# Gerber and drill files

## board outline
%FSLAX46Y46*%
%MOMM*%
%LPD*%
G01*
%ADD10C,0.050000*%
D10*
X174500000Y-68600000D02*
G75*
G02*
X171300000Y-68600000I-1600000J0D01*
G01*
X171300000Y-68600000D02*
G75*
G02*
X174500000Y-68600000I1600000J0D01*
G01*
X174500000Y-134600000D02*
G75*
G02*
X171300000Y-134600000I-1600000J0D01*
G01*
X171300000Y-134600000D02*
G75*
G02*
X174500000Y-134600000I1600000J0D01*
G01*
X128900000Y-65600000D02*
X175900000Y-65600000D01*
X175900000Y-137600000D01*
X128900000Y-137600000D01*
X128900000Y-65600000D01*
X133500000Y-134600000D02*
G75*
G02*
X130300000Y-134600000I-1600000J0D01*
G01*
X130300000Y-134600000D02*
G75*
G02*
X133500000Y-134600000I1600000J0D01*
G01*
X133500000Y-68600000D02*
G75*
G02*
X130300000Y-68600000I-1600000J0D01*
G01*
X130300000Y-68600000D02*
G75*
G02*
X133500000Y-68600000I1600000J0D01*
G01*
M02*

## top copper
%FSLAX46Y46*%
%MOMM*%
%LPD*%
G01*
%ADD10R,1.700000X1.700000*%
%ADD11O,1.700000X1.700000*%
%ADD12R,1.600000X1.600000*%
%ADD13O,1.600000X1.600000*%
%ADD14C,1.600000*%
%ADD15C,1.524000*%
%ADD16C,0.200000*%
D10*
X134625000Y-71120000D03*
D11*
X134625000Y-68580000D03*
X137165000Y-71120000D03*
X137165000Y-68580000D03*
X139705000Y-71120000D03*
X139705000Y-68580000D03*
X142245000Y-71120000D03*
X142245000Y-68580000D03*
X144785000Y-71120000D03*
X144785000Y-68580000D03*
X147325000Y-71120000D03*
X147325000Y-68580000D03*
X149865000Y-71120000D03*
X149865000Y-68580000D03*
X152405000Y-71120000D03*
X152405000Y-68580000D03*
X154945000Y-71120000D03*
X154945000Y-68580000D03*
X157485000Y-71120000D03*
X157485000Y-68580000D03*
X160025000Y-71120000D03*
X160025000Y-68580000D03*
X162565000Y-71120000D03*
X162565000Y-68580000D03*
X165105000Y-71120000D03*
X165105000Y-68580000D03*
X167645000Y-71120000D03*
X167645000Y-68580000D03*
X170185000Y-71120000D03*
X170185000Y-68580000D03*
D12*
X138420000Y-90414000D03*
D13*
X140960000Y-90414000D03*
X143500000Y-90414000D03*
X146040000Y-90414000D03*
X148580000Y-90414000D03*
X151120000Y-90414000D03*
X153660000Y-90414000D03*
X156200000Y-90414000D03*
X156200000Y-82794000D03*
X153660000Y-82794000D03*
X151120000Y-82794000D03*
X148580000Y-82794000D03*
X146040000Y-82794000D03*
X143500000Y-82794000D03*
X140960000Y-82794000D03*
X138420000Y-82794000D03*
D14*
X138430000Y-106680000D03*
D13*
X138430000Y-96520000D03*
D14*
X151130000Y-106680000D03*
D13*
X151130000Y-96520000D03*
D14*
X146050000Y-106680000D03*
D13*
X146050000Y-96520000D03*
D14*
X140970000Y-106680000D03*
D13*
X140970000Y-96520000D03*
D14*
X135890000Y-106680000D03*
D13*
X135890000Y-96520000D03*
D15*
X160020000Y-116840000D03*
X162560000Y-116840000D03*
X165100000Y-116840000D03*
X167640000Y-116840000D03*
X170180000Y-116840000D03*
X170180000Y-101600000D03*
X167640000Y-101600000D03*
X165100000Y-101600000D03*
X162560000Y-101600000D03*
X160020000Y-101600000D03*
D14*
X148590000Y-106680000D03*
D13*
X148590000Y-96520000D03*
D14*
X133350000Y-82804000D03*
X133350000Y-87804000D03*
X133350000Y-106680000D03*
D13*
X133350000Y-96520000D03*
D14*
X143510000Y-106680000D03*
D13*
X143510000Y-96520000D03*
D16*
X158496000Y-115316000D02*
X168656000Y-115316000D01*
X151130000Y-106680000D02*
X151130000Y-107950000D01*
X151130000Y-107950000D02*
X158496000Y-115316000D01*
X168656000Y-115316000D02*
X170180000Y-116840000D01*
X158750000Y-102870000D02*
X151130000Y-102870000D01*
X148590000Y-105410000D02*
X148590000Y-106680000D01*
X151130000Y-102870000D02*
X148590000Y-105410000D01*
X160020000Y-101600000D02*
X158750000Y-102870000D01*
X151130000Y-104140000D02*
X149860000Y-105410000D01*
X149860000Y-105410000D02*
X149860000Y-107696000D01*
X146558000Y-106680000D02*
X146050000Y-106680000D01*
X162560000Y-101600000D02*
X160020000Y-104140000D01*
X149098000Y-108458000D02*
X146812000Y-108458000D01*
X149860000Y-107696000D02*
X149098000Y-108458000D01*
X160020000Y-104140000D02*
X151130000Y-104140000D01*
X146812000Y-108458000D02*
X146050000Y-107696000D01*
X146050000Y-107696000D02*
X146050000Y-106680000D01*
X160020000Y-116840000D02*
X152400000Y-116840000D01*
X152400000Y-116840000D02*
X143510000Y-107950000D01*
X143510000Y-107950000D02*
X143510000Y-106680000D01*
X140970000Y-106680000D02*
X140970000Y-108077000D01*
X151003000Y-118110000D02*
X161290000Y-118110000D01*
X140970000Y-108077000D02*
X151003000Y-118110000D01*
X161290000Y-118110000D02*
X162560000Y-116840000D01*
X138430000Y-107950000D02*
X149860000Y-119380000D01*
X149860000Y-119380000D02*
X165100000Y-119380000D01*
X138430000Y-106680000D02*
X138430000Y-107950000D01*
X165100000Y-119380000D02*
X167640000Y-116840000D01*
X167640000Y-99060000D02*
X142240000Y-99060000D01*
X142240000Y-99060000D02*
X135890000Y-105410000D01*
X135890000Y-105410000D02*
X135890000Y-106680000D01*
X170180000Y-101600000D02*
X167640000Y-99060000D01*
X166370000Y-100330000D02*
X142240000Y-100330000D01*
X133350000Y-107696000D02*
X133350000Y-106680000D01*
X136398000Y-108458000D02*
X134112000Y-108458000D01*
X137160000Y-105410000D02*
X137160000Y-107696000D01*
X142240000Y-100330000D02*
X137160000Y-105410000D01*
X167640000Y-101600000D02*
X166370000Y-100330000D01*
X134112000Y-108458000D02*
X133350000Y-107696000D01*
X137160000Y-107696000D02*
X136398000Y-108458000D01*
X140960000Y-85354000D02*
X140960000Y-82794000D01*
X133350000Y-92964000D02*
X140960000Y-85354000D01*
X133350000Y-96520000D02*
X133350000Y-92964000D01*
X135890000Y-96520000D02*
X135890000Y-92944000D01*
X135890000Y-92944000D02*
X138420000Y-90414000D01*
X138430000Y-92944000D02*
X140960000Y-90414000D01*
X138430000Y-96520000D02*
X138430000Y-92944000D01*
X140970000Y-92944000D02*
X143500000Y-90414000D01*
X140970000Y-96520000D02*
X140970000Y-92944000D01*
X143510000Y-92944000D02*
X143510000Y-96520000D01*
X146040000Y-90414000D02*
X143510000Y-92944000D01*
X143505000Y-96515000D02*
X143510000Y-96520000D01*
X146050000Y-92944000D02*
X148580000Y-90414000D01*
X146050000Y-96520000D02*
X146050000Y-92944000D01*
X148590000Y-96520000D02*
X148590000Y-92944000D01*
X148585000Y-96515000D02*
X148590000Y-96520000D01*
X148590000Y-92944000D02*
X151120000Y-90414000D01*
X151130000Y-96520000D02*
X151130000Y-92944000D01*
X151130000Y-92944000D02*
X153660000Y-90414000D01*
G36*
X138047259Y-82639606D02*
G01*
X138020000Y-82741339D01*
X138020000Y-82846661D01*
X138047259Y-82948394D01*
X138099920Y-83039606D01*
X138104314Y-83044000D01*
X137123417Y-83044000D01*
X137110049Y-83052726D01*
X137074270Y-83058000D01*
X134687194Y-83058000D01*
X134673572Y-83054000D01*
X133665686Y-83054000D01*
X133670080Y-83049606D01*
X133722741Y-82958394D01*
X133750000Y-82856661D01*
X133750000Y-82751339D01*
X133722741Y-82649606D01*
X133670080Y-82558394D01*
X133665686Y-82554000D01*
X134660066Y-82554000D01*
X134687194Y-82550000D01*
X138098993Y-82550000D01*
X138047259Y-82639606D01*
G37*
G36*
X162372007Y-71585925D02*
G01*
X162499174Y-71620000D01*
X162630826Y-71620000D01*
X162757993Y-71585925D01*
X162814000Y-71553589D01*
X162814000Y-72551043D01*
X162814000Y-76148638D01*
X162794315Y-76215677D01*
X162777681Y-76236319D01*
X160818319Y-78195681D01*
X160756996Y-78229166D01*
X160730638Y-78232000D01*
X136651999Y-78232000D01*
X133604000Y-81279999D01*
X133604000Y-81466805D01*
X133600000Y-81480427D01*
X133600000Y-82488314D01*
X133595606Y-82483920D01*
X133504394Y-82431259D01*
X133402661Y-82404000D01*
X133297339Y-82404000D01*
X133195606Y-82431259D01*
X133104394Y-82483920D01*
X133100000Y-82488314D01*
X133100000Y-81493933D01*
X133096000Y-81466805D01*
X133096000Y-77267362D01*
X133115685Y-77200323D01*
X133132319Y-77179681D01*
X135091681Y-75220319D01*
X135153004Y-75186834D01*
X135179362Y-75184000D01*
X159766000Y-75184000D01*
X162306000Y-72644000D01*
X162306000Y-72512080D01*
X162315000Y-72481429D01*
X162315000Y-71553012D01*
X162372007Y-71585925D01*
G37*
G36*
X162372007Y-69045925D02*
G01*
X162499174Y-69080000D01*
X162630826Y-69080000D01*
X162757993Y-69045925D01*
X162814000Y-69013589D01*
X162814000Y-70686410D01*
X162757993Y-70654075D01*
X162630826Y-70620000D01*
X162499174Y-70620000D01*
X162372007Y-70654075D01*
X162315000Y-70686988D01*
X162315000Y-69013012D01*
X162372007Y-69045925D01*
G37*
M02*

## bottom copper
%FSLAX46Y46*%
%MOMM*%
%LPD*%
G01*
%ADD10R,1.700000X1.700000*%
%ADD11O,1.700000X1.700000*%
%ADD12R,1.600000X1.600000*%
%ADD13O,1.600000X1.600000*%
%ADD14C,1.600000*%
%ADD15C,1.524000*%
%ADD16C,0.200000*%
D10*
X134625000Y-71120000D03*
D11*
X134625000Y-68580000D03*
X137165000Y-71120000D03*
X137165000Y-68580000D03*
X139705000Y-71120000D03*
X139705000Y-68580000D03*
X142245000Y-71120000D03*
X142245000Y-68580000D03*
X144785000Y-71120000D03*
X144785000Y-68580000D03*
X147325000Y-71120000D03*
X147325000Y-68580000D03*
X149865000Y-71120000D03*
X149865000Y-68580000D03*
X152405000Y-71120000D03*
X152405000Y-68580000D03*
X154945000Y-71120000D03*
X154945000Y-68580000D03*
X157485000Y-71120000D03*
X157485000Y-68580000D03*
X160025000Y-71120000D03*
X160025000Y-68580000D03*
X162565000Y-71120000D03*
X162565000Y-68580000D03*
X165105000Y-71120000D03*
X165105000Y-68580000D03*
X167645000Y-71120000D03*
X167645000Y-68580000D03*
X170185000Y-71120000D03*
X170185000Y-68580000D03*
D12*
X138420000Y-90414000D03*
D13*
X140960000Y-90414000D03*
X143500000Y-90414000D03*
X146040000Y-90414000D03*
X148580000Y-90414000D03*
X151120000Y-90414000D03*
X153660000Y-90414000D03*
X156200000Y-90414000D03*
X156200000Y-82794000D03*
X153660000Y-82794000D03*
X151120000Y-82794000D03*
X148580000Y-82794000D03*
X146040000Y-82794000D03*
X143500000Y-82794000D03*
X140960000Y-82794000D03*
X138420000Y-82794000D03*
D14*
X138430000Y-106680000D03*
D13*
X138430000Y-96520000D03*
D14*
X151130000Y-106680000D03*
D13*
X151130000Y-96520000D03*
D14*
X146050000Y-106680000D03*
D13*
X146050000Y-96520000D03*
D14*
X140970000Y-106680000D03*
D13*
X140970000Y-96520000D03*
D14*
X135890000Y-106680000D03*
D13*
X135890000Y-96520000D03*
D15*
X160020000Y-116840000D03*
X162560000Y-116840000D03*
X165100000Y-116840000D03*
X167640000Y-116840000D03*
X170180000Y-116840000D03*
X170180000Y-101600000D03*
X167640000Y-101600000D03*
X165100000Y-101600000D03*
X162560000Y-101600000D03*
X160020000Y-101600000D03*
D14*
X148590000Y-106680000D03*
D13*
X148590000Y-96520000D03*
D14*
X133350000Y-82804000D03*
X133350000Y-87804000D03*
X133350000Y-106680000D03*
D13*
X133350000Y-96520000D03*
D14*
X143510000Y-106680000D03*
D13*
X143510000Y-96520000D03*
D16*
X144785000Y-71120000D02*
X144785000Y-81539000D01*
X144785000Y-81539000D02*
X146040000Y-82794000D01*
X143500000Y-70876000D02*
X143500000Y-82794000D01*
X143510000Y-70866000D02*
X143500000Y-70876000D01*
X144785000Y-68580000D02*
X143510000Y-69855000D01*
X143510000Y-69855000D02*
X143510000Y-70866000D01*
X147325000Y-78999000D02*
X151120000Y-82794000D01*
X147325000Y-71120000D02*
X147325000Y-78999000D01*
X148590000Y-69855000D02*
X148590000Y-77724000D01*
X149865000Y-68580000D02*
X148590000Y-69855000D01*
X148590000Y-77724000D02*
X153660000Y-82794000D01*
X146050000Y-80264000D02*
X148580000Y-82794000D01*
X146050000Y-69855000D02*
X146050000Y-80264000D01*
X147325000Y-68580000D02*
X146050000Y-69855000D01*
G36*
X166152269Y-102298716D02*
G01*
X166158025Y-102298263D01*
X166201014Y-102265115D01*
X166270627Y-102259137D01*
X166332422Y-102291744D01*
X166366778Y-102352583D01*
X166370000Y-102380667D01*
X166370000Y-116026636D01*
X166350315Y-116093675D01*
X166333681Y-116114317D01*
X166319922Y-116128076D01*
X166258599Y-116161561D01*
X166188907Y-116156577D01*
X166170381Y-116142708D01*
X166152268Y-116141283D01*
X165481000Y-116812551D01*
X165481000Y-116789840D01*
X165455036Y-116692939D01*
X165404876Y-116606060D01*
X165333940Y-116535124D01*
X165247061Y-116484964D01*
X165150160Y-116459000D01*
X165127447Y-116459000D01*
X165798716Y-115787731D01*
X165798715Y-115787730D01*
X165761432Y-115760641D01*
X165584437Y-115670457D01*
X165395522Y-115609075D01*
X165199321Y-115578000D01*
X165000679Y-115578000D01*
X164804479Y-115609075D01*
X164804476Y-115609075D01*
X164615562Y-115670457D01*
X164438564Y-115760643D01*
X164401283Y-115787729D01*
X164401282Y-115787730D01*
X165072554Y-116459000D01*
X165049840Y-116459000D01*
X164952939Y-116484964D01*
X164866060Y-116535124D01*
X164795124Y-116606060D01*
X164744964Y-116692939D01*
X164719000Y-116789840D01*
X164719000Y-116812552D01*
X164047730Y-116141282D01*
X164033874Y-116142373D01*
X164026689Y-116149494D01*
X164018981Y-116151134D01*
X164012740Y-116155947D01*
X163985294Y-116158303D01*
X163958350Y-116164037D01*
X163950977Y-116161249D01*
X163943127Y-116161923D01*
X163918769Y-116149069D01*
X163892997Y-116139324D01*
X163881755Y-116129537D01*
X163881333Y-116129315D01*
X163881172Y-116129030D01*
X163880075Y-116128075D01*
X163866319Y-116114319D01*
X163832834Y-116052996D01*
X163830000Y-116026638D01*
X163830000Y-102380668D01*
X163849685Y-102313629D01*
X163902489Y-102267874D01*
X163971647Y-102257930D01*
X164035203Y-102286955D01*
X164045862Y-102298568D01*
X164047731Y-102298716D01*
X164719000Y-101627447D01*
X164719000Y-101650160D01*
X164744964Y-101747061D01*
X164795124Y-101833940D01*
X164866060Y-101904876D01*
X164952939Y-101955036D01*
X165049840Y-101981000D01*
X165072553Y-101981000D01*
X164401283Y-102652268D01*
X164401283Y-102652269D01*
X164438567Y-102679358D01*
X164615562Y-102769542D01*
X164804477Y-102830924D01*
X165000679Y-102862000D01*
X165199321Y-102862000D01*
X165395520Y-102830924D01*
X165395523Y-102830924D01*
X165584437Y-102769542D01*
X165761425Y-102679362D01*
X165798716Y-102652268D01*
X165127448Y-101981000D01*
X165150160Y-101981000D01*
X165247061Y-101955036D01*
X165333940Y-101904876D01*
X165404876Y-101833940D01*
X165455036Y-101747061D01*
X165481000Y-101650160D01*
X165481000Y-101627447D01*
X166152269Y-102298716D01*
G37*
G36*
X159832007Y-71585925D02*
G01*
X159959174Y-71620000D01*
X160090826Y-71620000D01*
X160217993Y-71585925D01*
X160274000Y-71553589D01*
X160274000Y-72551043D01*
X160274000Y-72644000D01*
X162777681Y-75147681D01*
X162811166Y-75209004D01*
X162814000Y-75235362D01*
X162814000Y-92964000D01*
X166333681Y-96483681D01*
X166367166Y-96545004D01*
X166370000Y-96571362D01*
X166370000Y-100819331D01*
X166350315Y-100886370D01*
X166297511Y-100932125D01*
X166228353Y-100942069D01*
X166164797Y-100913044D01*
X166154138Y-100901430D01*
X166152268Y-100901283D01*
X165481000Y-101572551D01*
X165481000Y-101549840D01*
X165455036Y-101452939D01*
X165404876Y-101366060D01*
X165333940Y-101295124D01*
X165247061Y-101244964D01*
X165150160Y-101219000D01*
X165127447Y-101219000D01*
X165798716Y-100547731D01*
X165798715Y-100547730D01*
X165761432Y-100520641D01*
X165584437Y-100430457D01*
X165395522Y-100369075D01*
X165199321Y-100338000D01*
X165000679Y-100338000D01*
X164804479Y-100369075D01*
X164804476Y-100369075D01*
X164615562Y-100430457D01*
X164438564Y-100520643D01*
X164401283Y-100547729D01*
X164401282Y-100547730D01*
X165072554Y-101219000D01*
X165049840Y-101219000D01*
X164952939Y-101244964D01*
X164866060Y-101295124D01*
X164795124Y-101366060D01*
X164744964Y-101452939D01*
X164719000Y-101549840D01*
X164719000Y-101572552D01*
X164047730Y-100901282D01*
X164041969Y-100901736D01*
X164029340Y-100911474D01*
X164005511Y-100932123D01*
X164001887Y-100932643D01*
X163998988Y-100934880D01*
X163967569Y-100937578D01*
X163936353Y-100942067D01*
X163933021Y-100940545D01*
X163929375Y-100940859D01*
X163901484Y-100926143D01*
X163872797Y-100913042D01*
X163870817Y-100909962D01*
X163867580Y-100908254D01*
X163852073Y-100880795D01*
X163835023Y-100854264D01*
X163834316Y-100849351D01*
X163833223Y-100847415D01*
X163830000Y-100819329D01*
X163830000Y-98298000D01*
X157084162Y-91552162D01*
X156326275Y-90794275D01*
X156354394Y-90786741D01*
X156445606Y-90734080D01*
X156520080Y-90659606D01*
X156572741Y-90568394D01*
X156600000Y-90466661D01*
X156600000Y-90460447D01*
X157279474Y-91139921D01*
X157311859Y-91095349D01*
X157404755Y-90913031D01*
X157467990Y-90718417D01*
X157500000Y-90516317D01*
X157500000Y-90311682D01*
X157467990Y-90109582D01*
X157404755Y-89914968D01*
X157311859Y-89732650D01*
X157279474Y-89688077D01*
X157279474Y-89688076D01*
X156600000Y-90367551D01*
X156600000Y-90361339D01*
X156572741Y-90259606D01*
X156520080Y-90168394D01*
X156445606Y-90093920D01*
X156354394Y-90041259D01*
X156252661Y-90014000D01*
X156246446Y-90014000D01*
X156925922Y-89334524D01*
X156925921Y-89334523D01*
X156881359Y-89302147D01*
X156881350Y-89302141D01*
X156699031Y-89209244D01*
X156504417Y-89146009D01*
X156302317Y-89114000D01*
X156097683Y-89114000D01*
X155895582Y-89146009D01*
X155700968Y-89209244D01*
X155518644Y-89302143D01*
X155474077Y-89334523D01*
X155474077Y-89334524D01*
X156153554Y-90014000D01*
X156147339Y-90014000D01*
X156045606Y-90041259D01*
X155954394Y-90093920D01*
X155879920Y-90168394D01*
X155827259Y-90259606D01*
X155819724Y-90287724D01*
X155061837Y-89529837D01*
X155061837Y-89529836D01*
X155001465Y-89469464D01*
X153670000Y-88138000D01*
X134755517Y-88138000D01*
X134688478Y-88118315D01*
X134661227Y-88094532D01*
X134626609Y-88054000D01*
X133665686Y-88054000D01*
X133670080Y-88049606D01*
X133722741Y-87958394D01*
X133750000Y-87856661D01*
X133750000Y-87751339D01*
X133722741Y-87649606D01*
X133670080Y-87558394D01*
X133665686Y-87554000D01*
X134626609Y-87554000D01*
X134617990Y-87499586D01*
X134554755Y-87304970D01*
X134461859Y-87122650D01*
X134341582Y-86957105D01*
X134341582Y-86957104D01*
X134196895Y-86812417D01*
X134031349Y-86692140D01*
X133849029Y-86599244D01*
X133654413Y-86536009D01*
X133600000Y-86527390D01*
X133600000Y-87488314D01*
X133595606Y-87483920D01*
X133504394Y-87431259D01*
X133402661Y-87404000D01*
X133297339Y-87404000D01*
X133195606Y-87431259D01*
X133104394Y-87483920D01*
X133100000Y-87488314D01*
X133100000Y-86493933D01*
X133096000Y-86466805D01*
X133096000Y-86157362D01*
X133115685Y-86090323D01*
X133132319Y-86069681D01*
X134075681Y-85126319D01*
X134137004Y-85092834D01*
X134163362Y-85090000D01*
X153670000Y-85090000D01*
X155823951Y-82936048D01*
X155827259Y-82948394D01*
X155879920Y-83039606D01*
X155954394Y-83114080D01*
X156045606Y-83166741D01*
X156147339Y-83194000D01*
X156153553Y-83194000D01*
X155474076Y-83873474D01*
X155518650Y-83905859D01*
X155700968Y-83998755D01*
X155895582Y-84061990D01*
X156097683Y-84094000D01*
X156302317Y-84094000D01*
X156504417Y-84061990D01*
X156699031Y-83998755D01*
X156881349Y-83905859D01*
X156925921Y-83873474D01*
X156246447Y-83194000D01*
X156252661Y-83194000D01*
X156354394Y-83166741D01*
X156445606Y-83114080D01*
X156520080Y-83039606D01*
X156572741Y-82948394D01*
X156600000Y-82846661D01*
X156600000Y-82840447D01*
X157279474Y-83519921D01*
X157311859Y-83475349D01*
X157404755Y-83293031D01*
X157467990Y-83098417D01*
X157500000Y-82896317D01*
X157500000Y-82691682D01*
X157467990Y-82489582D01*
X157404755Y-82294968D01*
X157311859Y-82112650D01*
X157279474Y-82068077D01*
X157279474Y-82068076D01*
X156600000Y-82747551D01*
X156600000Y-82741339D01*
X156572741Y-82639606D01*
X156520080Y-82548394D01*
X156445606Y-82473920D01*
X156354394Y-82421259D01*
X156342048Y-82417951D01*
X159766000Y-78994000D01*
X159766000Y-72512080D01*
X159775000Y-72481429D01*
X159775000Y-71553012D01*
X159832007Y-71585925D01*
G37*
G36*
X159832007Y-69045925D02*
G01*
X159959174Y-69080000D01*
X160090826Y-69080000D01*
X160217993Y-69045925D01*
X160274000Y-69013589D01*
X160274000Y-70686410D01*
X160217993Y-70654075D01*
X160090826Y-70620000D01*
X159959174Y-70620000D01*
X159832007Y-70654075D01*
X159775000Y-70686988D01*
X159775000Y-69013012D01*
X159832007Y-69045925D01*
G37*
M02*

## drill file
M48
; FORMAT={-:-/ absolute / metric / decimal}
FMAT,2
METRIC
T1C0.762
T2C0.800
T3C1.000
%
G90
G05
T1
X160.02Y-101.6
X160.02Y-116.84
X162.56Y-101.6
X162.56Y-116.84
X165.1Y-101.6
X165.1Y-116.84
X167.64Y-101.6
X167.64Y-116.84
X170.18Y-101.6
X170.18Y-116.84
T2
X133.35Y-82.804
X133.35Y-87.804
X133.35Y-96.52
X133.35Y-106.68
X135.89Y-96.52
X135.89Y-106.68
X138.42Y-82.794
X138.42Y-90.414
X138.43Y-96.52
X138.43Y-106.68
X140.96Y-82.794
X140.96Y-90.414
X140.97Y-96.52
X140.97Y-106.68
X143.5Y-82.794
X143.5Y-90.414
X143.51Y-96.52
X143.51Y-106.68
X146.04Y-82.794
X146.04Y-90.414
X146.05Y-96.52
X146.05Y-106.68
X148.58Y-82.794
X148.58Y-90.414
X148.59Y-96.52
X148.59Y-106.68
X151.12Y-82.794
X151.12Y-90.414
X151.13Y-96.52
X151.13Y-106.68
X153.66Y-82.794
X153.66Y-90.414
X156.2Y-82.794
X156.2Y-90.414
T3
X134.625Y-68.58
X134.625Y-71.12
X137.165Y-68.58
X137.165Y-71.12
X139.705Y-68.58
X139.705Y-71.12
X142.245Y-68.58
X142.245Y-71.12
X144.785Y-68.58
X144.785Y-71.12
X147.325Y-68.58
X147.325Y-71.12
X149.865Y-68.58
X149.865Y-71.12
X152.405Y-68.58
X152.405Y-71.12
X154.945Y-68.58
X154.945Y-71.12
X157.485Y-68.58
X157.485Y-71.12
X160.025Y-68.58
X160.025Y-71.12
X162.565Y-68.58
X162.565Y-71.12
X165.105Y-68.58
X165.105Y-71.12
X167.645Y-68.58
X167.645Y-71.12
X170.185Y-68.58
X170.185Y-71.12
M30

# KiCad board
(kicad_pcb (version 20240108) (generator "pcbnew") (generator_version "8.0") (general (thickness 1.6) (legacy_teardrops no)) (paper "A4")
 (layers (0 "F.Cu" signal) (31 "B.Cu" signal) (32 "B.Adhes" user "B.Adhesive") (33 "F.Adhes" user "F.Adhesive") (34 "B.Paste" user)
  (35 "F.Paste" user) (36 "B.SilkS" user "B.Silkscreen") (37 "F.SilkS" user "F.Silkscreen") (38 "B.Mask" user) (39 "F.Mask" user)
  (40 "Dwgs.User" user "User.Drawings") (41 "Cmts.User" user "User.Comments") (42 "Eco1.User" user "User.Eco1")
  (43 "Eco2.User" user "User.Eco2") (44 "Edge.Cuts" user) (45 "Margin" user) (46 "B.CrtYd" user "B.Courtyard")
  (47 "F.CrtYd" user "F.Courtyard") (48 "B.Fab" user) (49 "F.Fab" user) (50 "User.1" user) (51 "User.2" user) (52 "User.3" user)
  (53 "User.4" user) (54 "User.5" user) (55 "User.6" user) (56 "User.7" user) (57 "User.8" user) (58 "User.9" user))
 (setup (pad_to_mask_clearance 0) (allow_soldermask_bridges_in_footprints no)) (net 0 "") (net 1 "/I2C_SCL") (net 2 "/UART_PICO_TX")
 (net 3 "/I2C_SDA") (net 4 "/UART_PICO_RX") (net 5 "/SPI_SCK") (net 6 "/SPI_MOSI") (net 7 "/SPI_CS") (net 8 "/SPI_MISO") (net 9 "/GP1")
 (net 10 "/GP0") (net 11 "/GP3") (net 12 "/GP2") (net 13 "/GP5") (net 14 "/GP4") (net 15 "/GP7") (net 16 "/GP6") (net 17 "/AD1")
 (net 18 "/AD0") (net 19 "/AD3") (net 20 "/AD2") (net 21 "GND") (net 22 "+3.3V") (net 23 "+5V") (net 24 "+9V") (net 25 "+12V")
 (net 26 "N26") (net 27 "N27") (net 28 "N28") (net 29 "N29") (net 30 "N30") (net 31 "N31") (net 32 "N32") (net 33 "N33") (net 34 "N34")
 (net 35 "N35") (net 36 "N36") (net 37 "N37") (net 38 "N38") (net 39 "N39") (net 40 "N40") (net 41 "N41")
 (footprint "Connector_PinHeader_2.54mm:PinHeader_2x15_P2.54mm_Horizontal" (layer "F.Cu") (at 134.625 71.12 90)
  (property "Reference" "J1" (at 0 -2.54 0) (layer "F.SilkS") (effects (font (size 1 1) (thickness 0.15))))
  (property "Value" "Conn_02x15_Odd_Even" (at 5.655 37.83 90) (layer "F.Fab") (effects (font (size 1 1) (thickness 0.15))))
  (pad "1" thru_hole rect (at 0 0 90) (size 1.7 1.7) (drill 1) (layers "*.Cu" "*.Mask") (remove_unused_layers no) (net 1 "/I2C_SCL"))
  (pad "2" thru_hole oval (at 2.54 0 90) (size 1.7 1.7) (drill 1) (layers "*.Cu" "*.Mask") (remove_unused_layers no) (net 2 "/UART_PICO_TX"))
  (pad "3" thru_hole oval (at 0 2.54 90) (size 1.7 1.7) (drill 1) (layers "*.Cu" "*.Mask") (remove_unused_layers no) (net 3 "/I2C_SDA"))
  (pad "4" thru_hole oval (at 2.54 2.54 90) (size 1.7 1.7) (drill 1) (layers "*.Cu" "*.Mask") (remove_unused_layers no)
   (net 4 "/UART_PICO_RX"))
  (pad "5" thru_hole oval (at 0 5.08 90) (size 1.7 1.7) (drill 1) (layers "*.Cu" "*.Mask") (remove_unused_layers no) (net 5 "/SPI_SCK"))
  (pad "6" thru_hole oval (at 2.54 5.08 90) (size 1.7 1.7) (drill 1) (layers "*.Cu" "*.Mask") (remove_unused_layers no) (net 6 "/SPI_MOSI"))
  (pad "7" thru_hole oval (at 0 7.62 90) (size 1.7 1.7) (drill 1) (layers "*.Cu" "*.Mask") (remove_unused_layers no) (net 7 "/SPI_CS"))
  (pad "8" thru_hole oval (at 2.54 7.62 90) (size 1.7 1.7) (drill 1) (layers "*.Cu" "*.Mask") (remove_unused_layers no) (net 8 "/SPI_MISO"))
  (pad "9" thru_hole oval (at 0 10.16 90) (size 1.7 1.7) (drill 1) (layers "*.Cu" "*.Mask") (remove_unused_layers no) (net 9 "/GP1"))
  (pad "10" thru_hole oval (at 2.54 10.16 90) (size 1.7 1.7) (drill 1) (layers "*.Cu" "*.Mask") (remove_unused_layers no) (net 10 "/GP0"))
  (pad "11" thru_hole oval (at 0 12.7 90) (size 1.7 1.7) (drill 1) (layers "*.Cu" "*.Mask") (remove_unused_layers no) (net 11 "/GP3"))
  (pad "12" thru_hole oval (at 2.54 12.7 90) (size 1.7 1.7) (drill 1) (layers "*.Cu" "*.Mask") (remove_unused_layers no) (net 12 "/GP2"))
  (pad "13" thru_hole oval (at 0 15.24 90) (size 1.7 1.7) (drill 1) (layers "*.Cu" "*.Mask") (remove_unused_layers no) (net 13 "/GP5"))
  (pad "14" thru_hole oval (at 2.54 15.24 90) (size 1.7 1.7) (drill 1) (layers "*.Cu" "*.Mask") (remove_unused_layers no) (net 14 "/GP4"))
  (pad "15" thru_hole oval (at 0 17.78 90) (size 1.7 1.7) (drill 1) (layers "*.Cu" "*.Mask") (remove_unused_layers no) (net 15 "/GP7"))
  (pad "16" thru_hole oval (at 2.54 17.78 90) (size 1.7 1.7) (drill 1) (layers "*.Cu" "*.Mask") (remove_unused_layers no) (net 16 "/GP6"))
  (pad "17" thru_hole oval (at 0 20.32 90) (size 1.7 1.7) (drill 1) (layers "*.Cu" "*.Mask") (remove_unused_layers no) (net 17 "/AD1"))
  (pad "18" thru_hole oval (at 2.54 20.32 90) (size 1.7 1.7) (drill 1) (layers "*.Cu" "*.Mask") (remove_unused_layers no) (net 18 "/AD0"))
  (pad "19" thru_hole oval (at 0 22.86 90) (size 1.7 1.7) (drill 1) (layers "*.Cu" "*.Mask") (remove_unused_layers no) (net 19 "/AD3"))
  (pad "20" thru_hole oval (at 2.54 22.86 90) (size 1.7 1.7) (drill 1) (layers "*.Cu" "*.Mask") (remove_unused_layers no) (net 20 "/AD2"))
  (pad "21" thru_hole oval (at 0 25.4 90) (size 1.7 1.7) (drill 1) (layers "*.Cu" "*.Mask") (remove_unused_layers no) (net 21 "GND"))
  (pad "22" thru_hole oval (at 2.54 25.4 90) (size 1.7 1.7) (drill 1) (layers "*.Cu" "*.Mask") (remove_unused_layers no) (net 21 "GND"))
  (pad "23" thru_hole oval (at 0 27.94 90) (size 1.7 1.7) (drill 1) (layers "*.Cu" "*.Mask") (remove_unused_layers no) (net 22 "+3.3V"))
  (pad "24" thru_hole oval (at 2.54 27.94 90) (size 1.7 1.7) (drill 1) (layers "*.Cu" "*.Mask") (remove_unused_layers no) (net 22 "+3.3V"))
  (pad "25" thru_hole oval (at 0 30.48 90) (size 1.7 1.7) (drill 1) (layers "*.Cu" "*.Mask") (remove_unused_layers no) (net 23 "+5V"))
  (pad "26" thru_hole oval (at 2.54 30.48 90) (size 1.7 1.7) (drill 1) (layers "*.Cu" "*.Mask") (remove_unused_layers no) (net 23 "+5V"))
  (pad "27" thru_hole oval (at 0 33.02 90) (size 1.7 1.7) (drill 1) (layers "*.Cu" "*.Mask") (remove_unused_layers no) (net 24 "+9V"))
  (pad "28" thru_hole oval (at 2.54 33.02 90) (size 1.7 1.7) (drill 1) (layers "*.Cu" "*.Mask") (remove_unused_layers no) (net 24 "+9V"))
  (pad "29" thru_hole oval (at 0 35.56 90) (size 1.7 1.7) (drill 1) (layers "*.Cu" "*.Mask") (remove_unused_layers no) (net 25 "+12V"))
  (pad "30" thru_hole oval (at 2.54 35.56 90) (size 1.7 1.7) (drill 1) (layers "*.Cu" "*.Mask") (remove_unused_layers no) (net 25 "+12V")))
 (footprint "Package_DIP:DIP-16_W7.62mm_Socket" (layer "F.Cu") (at 138.42 90.414 90)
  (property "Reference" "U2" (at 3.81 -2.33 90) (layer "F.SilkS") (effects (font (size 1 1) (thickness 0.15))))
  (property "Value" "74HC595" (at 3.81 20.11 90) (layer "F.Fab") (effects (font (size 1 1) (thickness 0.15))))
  (pad "1" thru_hole rect (at 0 0 90) (size 1.6 1.6) (drill 0.8) (layers "*.Cu" "*.Mask") (remove_unused_layers no) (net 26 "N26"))
  (pad "2" thru_hole oval (at 0 2.54 90) (size 1.6 1.6) (drill 0.8) (layers "*.Cu" "*.Mask") (remove_unused_layers no) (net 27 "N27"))
  (pad "3" thru_hole oval (at 0 5.08 90) (size 1.6 1.6) (drill 0.8) (layers "*.Cu" "*.Mask") (remove_unused_layers no) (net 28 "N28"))
  (pad "4" thru_hole oval (at 0 7.62 90) (size 1.6 1.6) (drill 0.8) (layers "*.Cu" "*.Mask") (remove_unused_layers no) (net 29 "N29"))
  (pad "5" thru_hole oval (at 0 10.16 90) (size 1.6 1.6) (drill 0.8) (layers "*.Cu" "*.Mask") (remove_unused_layers no) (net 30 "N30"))
  (pad "6" thru_hole oval (at 0 12.7 90) (size 1.6 1.6) (drill 0.8) (layers "*.Cu" "*.Mask") (remove_unused_layers no) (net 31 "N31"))
  (pad "7" thru_hole oval (at 0 15.24 90) (size 1.6 1.6) (drill 0.8) (layers "*.Cu" "*.Mask") (remove_unused_layers no) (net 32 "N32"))
  (pad "8" thru_hole oval (at 0 17.78 90) (size 1.6 1.6) (drill 0.8) (layers "*.Cu" "*.Mask") (remove_unused_layers no) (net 21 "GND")
   (thermal_bridge_angle 45))
  (pad "9" thru_hole oval (at 7.62 17.78 90) (size 1.6 1.6) (drill 0.8) (layers "*.Cu" "*.Mask") (remove_unused_layers no) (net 21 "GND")
   (thermal_bridge_angle 45))
  (pad "10" thru_hole oval (at 7.62 15.24 90) (size 1.6 1.6) (drill 0.8) (layers "*.Cu" "*.Mask") (remove_unused_layers no) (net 14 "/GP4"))
  (pad "11" thru_hole oval (at 7.62 12.7 90) (size 1.6 1.6) (drill 0.8) (layers "*.Cu" "*.Mask") (remove_unused_layers no) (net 11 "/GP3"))
  (pad "12" thru_hole oval (at 7.62 10.16 90) (size 1.6 1.6) (drill 0.8) (layers "*.Cu" "*.Mask") (remove_unused_layers no) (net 12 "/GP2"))
  (pad "13" thru_hole oval (at 7.62 7.62 90) (size 1.6 1.6) (drill 0.8) (layers "*.Cu" "*.Mask") (remove_unused_layers no) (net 9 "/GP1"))
  (pad "14" thru_hole oval (at 7.62 5.08 90) (size 1.6 1.6) (drill 0.8) (layers "*.Cu" "*.Mask") (remove_unused_layers no) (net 10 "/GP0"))
  (pad "15" thru_hole oval (at 7.62 2.54 90) (size 1.6 1.6) (drill 0.8) (layers "*.Cu" "*.Mask") (remove_unused_layers no) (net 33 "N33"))
  (pad "16" thru_hole oval (at 7.62 0 90) (size 1.6 1.6) (drill 0.8) (layers "*.Cu" "*.Mask") (remove_unused_layers no) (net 22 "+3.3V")
   (thermal_bridge_angle 0)))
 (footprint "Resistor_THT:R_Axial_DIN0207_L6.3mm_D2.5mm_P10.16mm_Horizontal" (layer "F.Cu") (at 138.43 106.68 90)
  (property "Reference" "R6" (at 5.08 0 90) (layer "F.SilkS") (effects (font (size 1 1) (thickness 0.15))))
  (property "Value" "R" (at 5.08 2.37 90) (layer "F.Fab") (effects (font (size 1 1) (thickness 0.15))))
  (pad "1" thru_hole circle (at 0 0 90) (size 1.6 1.6) (drill 0.8) (layers "*.Cu" "*.Mask") (remove_unused_layers no) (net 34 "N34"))
  (pad "2" thru_hole oval (at 10.16 0 90) (size 1.6 1.6) (drill 0.8) (layers "*.Cu" "*.Mask") (remove_unused_layers no) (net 27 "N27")))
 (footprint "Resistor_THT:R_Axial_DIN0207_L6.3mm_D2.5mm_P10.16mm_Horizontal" (layer "F.Cu") (at 151.13 106.68 90)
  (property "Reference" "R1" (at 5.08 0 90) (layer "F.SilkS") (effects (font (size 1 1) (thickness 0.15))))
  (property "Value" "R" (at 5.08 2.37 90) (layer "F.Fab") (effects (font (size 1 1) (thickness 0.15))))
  (pad "1" thru_hole circle (at 0 0 90) (size 1.6 1.6) (drill 0.8) (layers "*.Cu" "*.Mask") (remove_unused_layers no) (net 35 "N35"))
  (pad "2" thru_hole oval (at 10.16 0 90) (size 1.6 1.6) (drill 0.8) (layers "*.Cu" "*.Mask") (remove_unused_layers no) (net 32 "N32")))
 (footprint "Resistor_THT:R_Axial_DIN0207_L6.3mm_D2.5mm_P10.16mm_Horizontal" (layer "F.Cu") (at 146.05 106.68 90)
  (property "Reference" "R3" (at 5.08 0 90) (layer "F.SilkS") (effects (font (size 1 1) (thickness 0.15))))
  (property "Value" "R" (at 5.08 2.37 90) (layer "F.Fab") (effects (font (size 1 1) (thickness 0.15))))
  (pad "1" thru_hole circle (at 0 0 90) (size 1.6 1.6) (drill 0.8) (layers "*.Cu" "*.Mask") (remove_unused_layers no) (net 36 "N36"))
  (pad "2" thru_hole oval (at 10.16 0 90) (size 1.6 1.6) (drill 0.8) (layers "*.Cu" "*.Mask") (remove_unused_layers no) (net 30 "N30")))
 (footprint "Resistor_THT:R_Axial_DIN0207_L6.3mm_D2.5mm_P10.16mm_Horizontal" (layer "F.Cu") (at 140.97 106.68 90)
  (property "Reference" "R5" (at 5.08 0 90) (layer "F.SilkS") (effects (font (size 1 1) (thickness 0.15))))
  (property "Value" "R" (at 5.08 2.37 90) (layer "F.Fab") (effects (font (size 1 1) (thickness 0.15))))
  (pad "1" thru_hole circle (at 0 0 90) (size 1.6 1.6) (drill 0.8) (layers "*.Cu" "*.Mask") (remove_unused_layers no) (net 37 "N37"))
  (pad "2" thru_hole oval (at 10.16 0 90) (size 1.6 1.6) (drill 0.8) (layers "*.Cu" "*.Mask") (remove_unused_layers no) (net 28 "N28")))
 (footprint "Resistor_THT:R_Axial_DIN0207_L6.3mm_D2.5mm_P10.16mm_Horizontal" (layer "F.Cu") (at 135.89 106.68 90)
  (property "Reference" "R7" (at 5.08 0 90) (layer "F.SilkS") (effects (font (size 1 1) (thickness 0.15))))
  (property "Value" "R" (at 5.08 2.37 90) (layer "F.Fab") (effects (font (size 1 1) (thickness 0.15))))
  (pad "1" thru_hole circle (at 0 0 90) (size 1.6 1.6) (drill 0.8) (layers "*.Cu" "*.Mask") (remove_unused_layers no) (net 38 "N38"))
  (pad "2" thru_hole oval (at 10.16 0 90) (size 1.6 1.6) (drill 0.8) (layers "*.Cu" "*.Mask") (remove_unused_layers no) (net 26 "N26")))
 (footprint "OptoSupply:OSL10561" (layer "F.Cu") (at 165.1 109.22)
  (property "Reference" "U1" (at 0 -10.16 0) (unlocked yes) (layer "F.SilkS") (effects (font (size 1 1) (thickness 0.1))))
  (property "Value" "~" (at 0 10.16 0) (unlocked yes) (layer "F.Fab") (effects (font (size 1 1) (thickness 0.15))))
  (pad "1" thru_hole circle (at -5.08 7.62) (size 1.524 1.524) (drill 0.762) (layers "*.Cu" "*.Mask") (remove_unused_layers no)
   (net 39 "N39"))
  (pad "2" thru_hole circle (at -2.54 7.62) (size 1.524 1.524) (drill 0.762) (layers "*.Cu" "*.Mask") (remove_unused_layers no)
   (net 37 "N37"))
  (pad "3" thru_hole circle (at 0 7.62) (size 1.524 1.524) (drill 0.762) (layers "*.Cu" "*.Mask") (remove_unused_layers no) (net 21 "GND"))
  (pad "4" thru_hole circle (at 2.54 7.62) (size 1.524 1.524) (drill 0.762) (layers "*.Cu" "*.Mask") (remove_unused_layers no)
   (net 34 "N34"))
  (pad "5" thru_hole circle (at 5.08 7.62) (size 1.524 1.524) (drill 0.762) (layers "*.Cu" "*.Mask") (remove_unused_layers no)
   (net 35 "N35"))
  (pad "6" thru_hole circle (at 5.08 -7.62) (size 1.524 1.524) (drill 0.762) (layers "*.Cu" "*.Mask") (remove_unused_layers no)
   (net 38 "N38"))
  (pad "7" thru_hole circle (at 2.54 -7.62) (size 1.524 1.524) (drill 0.762) (layers "*.Cu" "*.Mask") (remove_unused_layers no)
   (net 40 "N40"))
  (pad "8" thru_hole circle (at 0 -7.62) (size 1.524 1.524) (drill 0.762) (layers "*.Cu" "*.Mask") (remove_unused_layers no) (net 21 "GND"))
  (pad "9" thru_hole circle (at -2.54 -7.62) (size 1.524 1.524) (drill 0.762) (layers "*.Cu" "*.Mask") (remove_unused_layers no)
   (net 36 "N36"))
  (pad "10" thru_hole circle (at -5.08 -7.62) (size 1.524 1.524) (drill 0.762) (layers "*.Cu" "*.Mask") (remove_unused_layers no)
   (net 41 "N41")))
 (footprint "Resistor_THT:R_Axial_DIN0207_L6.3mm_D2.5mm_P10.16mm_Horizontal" (layer "F.Cu") (at 148.59 106.68 90)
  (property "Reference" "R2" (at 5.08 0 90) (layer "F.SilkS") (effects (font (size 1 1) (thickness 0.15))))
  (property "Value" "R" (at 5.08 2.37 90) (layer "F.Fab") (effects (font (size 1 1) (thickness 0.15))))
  (pad "1" thru_hole circle (at 0 0 90) (size 1.6 1.6) (drill 0.8) (layers "*.Cu" "*.Mask") (remove_unused_layers no) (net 41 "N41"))
  (pad "2" thru_hole oval (at 10.16 0 90) (size 1.6 1.6) (drill 0.8) (layers "*.Cu" "*.Mask") (remove_unused_layers no) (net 31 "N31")))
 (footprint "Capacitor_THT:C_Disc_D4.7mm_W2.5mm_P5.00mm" (layer "F.Cu") (at 133.35 82.804 -90)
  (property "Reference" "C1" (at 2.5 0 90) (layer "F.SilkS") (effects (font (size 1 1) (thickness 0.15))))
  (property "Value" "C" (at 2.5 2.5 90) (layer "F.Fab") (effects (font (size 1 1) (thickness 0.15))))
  (pad "1" thru_hole circle (at 0 0 270) (size 1.6 1.6) (drill 0.8) (layers "*.Cu" "*.Mask") (remove_unused_layers no) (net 22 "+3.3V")
   (thermal_bridge_angle 0))
  (pad "2" thru_hole circle (at 5 0 270) (size 1.6 1.6) (drill 0.8) (layers "*.Cu" "*.Mask") (remove_unused_layers no) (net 21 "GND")
   (thermal_bridge_angle 0)))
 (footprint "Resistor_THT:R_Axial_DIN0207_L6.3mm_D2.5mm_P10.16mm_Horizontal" (layer "F.Cu") (at 133.35 106.68 90)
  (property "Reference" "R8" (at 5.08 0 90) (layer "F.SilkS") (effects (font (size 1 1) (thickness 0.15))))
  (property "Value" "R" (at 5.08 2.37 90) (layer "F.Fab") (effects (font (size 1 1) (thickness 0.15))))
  (pad "1" thru_hole circle (at 0 0 90) (size 1.6 1.6) (drill 0.8) (layers "*.Cu" "*.Mask") (remove_unused_layers no) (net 40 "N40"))
  (pad "2" thru_hole oval (at 10.16 0 90) (size 1.6 1.6) (drill 0.8) (layers "*.Cu" "*.Mask") (remove_unused_layers no) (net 33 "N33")))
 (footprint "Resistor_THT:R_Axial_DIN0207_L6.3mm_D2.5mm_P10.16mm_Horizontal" (layer "F.Cu") (at 143.51 106.68 90)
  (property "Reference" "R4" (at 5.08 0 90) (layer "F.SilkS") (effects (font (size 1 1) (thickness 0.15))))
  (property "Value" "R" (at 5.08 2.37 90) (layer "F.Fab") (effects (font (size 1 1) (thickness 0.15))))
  (pad "1" thru_hole circle (at 0 0 90) (size 1.6 1.6) (drill 0.8) (layers "*.Cu" "*.Mask") (remove_unused_layers no) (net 39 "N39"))
  (pad "2" thru_hole oval (at 10.16 0 90) (size 1.6 1.6) (drill 0.8) (layers "*.Cu" "*.Mask") (remove_unused_layers no) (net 29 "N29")))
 (gr_circle (center 172.9 68.6) (end 172.9 70.2) (stroke (width 0.05) (type default)) (fill none) (layer "Edge.Cuts"))
 (gr_circle (center 172.9 134.6) (end 171.3 134.6) (stroke (width 0.05) (type default)) (fill none) (layer "Edge.Cuts"))
 (gr_rect (start 128.9 65.6) (end 175.9 137.6) (stroke (width 0.05) (type default)) (fill none) (layer "Edge.Cuts"))
 (gr_circle (center 131.9 134.6) (end 131.9 133) (stroke (width 0.05) (type default)) (fill none) (layer "Edge.Cuts"))
 (gr_circle (center 131.9 68.6) (end 133.5 68.6) (stroke (width 0.05) (type default)) (fill none) (layer "Edge.Cuts"))
 (segment (start 144.785 71.12) (end 144.785 81.539) (width 0.2) (layer "B.Cu") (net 9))
 (segment (start 144.785 81.539) (end 146.04 82.794) (width 0.2) (layer "B.Cu") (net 9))
 (segment (start 143.5 70.876) (end 143.5 82.794) (width 0.2) (layer "B.Cu") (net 10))
 (segment (start 143.51 70.866) (end 143.5 70.876) (width 0.2) (layer "B.Cu") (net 10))
 (segment (start 144.785 68.58) (end 143.51 69.855) (width 0.2) (layer "B.Cu") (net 10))
 (segment (start 143.51 69.855) (end 143.51 70.866) (width 0.2) (layer "B.Cu") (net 10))
 (segment (start 147.325 78.999) (end 151.12 82.794) (width 0.2) (layer "B.Cu") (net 11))
 (segment (start 147.325 71.12) (end 147.325 78.999) (width 0.2) (layer "B.Cu") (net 11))
 (segment (start 148.59 69.855) (end 148.59 77.724) (width 0.2) (layer "B.Cu") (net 14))
 (segment (start 149.865 68.58) (end 148.59 69.855) (width 0.2) (layer "B.Cu") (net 14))
 (segment (start 148.59 77.724) (end 153.66 82.794) (width 0.2) (layer "B.Cu") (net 14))
 (segment (start 146.05 80.264) (end 148.58 82.794) (width 0.2) (layer "B.Cu") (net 12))
 (segment (start 146.05 69.855) (end 146.05 80.264) (width 0.2) (layer "B.Cu") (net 12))
 (segment (start 147.325 68.58) (end 146.05 69.855) (width 0.2) (layer "B.Cu") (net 12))
 (segment (start 158.496 115.316) (end 168.656 115.316) (width 0.2) (layer "F.Cu") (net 35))
 (segment (start 151.13 106.68) (end 151.13 107.95) (width 0.2) (layer "F.Cu") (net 35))
 (segment (start 151.13 107.95) (end 158.496 115.316) (width 0.2) (layer "F.Cu") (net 35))
 (segment (start 168.656 115.316) (end 170.18 116.84) (width 0.2) (layer "F.Cu") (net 35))
 (segment (start 158.75 102.87) (end 151.13 102.87) (width 0.2) (layer "F.Cu") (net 41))
 (segment (start 148.59 105.41) (end 148.59 106.68) (width 0.2) (layer "F.Cu") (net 41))
 (segment (start 151.13 102.87) (end 148.59 105.41) (width 0.2) (layer "F.Cu") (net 41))
 (segment (start 160.02 101.6) (end 158.75 102.87) (width 0.2) (layer "F.Cu") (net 41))
 (segment (start 151.13 104.14) (end 149.86 105.41) (width 0.2) (layer "F.Cu") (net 36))
 (segment (start 149.86 105.41) (end 149.86 107.696) (width 0.2) (layer "F.Cu") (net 36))
 (segment (start 146.558 106.68) (end 146.05 106.68) (width 0.2) (layer "F.Cu") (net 36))
 (segment (start 162.56 101.6) (end 160.02 104.14) (width 0.2) (layer "F.Cu") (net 36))
 (segment (start 149.098 108.458) (end 146.812 108.458) (width 0.2) (layer "F.Cu") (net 36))
 (segment (start 149.86 107.696) (end 149.098 108.458) (width 0.2) (layer "F.Cu") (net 36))
 (segment (start 160.02 104.14) (end 151.13 104.14) (width 0.2) (layer "F.Cu") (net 36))
 (segment (start 146.812 108.458) (end 146.05 107.696) (width 0.2) (layer "F.Cu") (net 36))
 (segment (start 146.05 107.696) (end 146.05 106.68) (width 0.2) (layer "F.Cu") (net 36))
 (segment (start 160.02 116.84) (end 152.4 116.84) (width 0.2) (layer "F.Cu") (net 39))
 (segment (start 152.4 116.84) (end 143.51 107.95) (width 0.2) (layer "F.Cu") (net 39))
 (segment (start 143.51 107.95) (end 143.51 106.68) (width 0.2) (layer "F.Cu") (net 39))
 (segment (start 140.97 106.68) (end 140.97 108.077) (width 0.2) (layer "F.Cu") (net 37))
 (segment (start 151.003 118.11) (end 161.29 118.11) (width 0.2) (layer "F.Cu") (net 37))
 (segment (start 140.97 108.077) (end 151.003 118.11) (width 0.2) (layer "F.Cu") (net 37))
 (segment (start 161.29 118.11) (end 162.56 116.84) (width 0.2) (layer "F.Cu") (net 37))
 (segment (start 138.43 107.95) (end 149.86 119.38) (width 0.2) (layer "F.Cu") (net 34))
 (segment (start 149.86 119.38) (end 165.1 119.38) (width 0.2) (layer "F.Cu") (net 34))
 (segment (start 138.43 106.68) (end 138.43 107.95) (width 0.2) (layer "F.Cu") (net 34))
 (segment (start 165.1 119.38) (end 167.64 116.84) (width 0.2) (layer "F.Cu") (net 34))
 (segment (start 167.64 99.06) (end 142.24 99.06) (width 0.2) (layer "F.Cu") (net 38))
 (segment (start 142.24 99.06) (end 135.89 105.41) (width 0.2) (layer "F.Cu") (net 38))
 (segment (start 135.89 105.41) (end 135.89 106.68) (width 0.2) (layer "F.Cu") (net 38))
 (segment (start 170.18 101.6) (end 167.64 99.06) (width 0.2) (layer "F.Cu") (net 38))
 (segment (start 166.37 100.33) (end 142.24 100.33) (width 0.2) (layer "F.Cu") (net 40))
 (segment (start 133.35 107.696) (end 133.35 106.68) (width 0.2) (layer "F.Cu") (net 40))
 (segment (start 136.398 108.458) (end 134.112 108.458) (width 0.2) (layer "F.Cu") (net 40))
 (segment (start 137.16 105.41) (end 137.16 107.696) (width 0.2) (layer "F.Cu") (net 40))
 (segment (start 142.24 100.33) (end 137.16 105.41) (width 0.2) (layer "F.Cu") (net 40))
 (segment (start 167.64 101.6) (end 166.37 100.33) (width 0.2) (layer "F.Cu") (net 40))
 (segment (start 134.112 108.458) (end 133.35 107.696) (width 0.2) (layer "F.Cu") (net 40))
 (segment (start 137.16 107.696) (end 136.398 108.458) (width 0.2) (layer "F.Cu") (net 40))
 (segment (start 140.96 85.354) (end 140.96 82.794) (width 0.2) (layer "F.Cu") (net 33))
 (segment (start 133.35 92.964) (end 140.96 85.354) (width 0.2) (layer "F.Cu") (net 33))
 (segment (start 133.35 96.52) (end 133.35 92.964) (width 0.2) (layer "F.Cu") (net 33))
 (segment (start 135.89 96.52) (end 135.89 92.944) (width 0.2) (layer "F.Cu") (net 26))
 (segment (start 135.89 92.944) (end 138.42 90.414) (width 0.2) (layer "F.Cu") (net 26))
 (segment (start 138.43 92.944) (end 140.96 90.414) (width 0.2) (layer "F.Cu") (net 27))
 (segment (start 138.43 96.52) (end 138.43 92.944) (width 0.2) (layer "F.Cu") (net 27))
 (segment (start 140.97 92.944) (end 143.5 90.414) (width 0.2) (layer "F.Cu") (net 28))
 (segment (start 140.97 96.52) (end 140.97 92.944) (width 0.2) (layer "F.Cu") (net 28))
 (segment (start 143.51 92.944) (end 143.51 96.52) (width 0.2) (layer "F.Cu") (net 29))
 (segment (start 146.04 90.414) (end 143.51 92.944) (width 0.2) (layer "F.Cu") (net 29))
 (segment (start 143.505 96.515) (end 143.51 96.52) (width 0.2) (layer "F.Cu") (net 29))
 (segment (start 146.05 92.944) (end 148.58 90.414) (width 0.2) (layer "F.Cu") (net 30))
 (segment (start 146.05 96.52) (end 146.05 92.944) (width 0.2) (layer "F.Cu") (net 30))
 (segment (start 148.59 96.52) (end 148.59 92.944) (width 0.2) (layer "F.Cu") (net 31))
 (segment (start 148.585 96.515) (end 148.59 96.52) (width 0.2) (layer "F.Cu") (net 31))
 (segment (start 148.59 92.944) (end 151.12 90.414) (width 0.2) (layer "F.Cu") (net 31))
 (segment (start 151.13 96.52) (end 151.13 92.944) (width 0.2) (layer "F.Cu") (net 32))
 (segment (start 151.13 92.944) (end 153.66 90.414) (width 0.2) (layer "F.Cu") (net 32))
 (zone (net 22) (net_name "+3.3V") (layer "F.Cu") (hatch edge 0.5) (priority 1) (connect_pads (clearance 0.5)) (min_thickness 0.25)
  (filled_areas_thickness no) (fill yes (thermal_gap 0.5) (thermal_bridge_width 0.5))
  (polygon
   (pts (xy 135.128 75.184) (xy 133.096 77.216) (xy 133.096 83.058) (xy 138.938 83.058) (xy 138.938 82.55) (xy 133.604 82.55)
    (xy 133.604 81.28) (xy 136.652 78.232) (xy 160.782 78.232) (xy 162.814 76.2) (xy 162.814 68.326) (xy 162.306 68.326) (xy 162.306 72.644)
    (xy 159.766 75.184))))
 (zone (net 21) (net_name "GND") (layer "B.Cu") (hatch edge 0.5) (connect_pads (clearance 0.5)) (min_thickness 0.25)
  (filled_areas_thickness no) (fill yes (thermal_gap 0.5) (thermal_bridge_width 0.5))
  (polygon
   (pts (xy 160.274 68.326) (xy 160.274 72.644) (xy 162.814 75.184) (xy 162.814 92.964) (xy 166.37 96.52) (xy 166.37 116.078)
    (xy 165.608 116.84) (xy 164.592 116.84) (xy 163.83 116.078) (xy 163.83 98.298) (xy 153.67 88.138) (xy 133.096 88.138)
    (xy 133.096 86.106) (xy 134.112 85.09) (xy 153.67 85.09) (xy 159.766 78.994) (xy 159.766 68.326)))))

